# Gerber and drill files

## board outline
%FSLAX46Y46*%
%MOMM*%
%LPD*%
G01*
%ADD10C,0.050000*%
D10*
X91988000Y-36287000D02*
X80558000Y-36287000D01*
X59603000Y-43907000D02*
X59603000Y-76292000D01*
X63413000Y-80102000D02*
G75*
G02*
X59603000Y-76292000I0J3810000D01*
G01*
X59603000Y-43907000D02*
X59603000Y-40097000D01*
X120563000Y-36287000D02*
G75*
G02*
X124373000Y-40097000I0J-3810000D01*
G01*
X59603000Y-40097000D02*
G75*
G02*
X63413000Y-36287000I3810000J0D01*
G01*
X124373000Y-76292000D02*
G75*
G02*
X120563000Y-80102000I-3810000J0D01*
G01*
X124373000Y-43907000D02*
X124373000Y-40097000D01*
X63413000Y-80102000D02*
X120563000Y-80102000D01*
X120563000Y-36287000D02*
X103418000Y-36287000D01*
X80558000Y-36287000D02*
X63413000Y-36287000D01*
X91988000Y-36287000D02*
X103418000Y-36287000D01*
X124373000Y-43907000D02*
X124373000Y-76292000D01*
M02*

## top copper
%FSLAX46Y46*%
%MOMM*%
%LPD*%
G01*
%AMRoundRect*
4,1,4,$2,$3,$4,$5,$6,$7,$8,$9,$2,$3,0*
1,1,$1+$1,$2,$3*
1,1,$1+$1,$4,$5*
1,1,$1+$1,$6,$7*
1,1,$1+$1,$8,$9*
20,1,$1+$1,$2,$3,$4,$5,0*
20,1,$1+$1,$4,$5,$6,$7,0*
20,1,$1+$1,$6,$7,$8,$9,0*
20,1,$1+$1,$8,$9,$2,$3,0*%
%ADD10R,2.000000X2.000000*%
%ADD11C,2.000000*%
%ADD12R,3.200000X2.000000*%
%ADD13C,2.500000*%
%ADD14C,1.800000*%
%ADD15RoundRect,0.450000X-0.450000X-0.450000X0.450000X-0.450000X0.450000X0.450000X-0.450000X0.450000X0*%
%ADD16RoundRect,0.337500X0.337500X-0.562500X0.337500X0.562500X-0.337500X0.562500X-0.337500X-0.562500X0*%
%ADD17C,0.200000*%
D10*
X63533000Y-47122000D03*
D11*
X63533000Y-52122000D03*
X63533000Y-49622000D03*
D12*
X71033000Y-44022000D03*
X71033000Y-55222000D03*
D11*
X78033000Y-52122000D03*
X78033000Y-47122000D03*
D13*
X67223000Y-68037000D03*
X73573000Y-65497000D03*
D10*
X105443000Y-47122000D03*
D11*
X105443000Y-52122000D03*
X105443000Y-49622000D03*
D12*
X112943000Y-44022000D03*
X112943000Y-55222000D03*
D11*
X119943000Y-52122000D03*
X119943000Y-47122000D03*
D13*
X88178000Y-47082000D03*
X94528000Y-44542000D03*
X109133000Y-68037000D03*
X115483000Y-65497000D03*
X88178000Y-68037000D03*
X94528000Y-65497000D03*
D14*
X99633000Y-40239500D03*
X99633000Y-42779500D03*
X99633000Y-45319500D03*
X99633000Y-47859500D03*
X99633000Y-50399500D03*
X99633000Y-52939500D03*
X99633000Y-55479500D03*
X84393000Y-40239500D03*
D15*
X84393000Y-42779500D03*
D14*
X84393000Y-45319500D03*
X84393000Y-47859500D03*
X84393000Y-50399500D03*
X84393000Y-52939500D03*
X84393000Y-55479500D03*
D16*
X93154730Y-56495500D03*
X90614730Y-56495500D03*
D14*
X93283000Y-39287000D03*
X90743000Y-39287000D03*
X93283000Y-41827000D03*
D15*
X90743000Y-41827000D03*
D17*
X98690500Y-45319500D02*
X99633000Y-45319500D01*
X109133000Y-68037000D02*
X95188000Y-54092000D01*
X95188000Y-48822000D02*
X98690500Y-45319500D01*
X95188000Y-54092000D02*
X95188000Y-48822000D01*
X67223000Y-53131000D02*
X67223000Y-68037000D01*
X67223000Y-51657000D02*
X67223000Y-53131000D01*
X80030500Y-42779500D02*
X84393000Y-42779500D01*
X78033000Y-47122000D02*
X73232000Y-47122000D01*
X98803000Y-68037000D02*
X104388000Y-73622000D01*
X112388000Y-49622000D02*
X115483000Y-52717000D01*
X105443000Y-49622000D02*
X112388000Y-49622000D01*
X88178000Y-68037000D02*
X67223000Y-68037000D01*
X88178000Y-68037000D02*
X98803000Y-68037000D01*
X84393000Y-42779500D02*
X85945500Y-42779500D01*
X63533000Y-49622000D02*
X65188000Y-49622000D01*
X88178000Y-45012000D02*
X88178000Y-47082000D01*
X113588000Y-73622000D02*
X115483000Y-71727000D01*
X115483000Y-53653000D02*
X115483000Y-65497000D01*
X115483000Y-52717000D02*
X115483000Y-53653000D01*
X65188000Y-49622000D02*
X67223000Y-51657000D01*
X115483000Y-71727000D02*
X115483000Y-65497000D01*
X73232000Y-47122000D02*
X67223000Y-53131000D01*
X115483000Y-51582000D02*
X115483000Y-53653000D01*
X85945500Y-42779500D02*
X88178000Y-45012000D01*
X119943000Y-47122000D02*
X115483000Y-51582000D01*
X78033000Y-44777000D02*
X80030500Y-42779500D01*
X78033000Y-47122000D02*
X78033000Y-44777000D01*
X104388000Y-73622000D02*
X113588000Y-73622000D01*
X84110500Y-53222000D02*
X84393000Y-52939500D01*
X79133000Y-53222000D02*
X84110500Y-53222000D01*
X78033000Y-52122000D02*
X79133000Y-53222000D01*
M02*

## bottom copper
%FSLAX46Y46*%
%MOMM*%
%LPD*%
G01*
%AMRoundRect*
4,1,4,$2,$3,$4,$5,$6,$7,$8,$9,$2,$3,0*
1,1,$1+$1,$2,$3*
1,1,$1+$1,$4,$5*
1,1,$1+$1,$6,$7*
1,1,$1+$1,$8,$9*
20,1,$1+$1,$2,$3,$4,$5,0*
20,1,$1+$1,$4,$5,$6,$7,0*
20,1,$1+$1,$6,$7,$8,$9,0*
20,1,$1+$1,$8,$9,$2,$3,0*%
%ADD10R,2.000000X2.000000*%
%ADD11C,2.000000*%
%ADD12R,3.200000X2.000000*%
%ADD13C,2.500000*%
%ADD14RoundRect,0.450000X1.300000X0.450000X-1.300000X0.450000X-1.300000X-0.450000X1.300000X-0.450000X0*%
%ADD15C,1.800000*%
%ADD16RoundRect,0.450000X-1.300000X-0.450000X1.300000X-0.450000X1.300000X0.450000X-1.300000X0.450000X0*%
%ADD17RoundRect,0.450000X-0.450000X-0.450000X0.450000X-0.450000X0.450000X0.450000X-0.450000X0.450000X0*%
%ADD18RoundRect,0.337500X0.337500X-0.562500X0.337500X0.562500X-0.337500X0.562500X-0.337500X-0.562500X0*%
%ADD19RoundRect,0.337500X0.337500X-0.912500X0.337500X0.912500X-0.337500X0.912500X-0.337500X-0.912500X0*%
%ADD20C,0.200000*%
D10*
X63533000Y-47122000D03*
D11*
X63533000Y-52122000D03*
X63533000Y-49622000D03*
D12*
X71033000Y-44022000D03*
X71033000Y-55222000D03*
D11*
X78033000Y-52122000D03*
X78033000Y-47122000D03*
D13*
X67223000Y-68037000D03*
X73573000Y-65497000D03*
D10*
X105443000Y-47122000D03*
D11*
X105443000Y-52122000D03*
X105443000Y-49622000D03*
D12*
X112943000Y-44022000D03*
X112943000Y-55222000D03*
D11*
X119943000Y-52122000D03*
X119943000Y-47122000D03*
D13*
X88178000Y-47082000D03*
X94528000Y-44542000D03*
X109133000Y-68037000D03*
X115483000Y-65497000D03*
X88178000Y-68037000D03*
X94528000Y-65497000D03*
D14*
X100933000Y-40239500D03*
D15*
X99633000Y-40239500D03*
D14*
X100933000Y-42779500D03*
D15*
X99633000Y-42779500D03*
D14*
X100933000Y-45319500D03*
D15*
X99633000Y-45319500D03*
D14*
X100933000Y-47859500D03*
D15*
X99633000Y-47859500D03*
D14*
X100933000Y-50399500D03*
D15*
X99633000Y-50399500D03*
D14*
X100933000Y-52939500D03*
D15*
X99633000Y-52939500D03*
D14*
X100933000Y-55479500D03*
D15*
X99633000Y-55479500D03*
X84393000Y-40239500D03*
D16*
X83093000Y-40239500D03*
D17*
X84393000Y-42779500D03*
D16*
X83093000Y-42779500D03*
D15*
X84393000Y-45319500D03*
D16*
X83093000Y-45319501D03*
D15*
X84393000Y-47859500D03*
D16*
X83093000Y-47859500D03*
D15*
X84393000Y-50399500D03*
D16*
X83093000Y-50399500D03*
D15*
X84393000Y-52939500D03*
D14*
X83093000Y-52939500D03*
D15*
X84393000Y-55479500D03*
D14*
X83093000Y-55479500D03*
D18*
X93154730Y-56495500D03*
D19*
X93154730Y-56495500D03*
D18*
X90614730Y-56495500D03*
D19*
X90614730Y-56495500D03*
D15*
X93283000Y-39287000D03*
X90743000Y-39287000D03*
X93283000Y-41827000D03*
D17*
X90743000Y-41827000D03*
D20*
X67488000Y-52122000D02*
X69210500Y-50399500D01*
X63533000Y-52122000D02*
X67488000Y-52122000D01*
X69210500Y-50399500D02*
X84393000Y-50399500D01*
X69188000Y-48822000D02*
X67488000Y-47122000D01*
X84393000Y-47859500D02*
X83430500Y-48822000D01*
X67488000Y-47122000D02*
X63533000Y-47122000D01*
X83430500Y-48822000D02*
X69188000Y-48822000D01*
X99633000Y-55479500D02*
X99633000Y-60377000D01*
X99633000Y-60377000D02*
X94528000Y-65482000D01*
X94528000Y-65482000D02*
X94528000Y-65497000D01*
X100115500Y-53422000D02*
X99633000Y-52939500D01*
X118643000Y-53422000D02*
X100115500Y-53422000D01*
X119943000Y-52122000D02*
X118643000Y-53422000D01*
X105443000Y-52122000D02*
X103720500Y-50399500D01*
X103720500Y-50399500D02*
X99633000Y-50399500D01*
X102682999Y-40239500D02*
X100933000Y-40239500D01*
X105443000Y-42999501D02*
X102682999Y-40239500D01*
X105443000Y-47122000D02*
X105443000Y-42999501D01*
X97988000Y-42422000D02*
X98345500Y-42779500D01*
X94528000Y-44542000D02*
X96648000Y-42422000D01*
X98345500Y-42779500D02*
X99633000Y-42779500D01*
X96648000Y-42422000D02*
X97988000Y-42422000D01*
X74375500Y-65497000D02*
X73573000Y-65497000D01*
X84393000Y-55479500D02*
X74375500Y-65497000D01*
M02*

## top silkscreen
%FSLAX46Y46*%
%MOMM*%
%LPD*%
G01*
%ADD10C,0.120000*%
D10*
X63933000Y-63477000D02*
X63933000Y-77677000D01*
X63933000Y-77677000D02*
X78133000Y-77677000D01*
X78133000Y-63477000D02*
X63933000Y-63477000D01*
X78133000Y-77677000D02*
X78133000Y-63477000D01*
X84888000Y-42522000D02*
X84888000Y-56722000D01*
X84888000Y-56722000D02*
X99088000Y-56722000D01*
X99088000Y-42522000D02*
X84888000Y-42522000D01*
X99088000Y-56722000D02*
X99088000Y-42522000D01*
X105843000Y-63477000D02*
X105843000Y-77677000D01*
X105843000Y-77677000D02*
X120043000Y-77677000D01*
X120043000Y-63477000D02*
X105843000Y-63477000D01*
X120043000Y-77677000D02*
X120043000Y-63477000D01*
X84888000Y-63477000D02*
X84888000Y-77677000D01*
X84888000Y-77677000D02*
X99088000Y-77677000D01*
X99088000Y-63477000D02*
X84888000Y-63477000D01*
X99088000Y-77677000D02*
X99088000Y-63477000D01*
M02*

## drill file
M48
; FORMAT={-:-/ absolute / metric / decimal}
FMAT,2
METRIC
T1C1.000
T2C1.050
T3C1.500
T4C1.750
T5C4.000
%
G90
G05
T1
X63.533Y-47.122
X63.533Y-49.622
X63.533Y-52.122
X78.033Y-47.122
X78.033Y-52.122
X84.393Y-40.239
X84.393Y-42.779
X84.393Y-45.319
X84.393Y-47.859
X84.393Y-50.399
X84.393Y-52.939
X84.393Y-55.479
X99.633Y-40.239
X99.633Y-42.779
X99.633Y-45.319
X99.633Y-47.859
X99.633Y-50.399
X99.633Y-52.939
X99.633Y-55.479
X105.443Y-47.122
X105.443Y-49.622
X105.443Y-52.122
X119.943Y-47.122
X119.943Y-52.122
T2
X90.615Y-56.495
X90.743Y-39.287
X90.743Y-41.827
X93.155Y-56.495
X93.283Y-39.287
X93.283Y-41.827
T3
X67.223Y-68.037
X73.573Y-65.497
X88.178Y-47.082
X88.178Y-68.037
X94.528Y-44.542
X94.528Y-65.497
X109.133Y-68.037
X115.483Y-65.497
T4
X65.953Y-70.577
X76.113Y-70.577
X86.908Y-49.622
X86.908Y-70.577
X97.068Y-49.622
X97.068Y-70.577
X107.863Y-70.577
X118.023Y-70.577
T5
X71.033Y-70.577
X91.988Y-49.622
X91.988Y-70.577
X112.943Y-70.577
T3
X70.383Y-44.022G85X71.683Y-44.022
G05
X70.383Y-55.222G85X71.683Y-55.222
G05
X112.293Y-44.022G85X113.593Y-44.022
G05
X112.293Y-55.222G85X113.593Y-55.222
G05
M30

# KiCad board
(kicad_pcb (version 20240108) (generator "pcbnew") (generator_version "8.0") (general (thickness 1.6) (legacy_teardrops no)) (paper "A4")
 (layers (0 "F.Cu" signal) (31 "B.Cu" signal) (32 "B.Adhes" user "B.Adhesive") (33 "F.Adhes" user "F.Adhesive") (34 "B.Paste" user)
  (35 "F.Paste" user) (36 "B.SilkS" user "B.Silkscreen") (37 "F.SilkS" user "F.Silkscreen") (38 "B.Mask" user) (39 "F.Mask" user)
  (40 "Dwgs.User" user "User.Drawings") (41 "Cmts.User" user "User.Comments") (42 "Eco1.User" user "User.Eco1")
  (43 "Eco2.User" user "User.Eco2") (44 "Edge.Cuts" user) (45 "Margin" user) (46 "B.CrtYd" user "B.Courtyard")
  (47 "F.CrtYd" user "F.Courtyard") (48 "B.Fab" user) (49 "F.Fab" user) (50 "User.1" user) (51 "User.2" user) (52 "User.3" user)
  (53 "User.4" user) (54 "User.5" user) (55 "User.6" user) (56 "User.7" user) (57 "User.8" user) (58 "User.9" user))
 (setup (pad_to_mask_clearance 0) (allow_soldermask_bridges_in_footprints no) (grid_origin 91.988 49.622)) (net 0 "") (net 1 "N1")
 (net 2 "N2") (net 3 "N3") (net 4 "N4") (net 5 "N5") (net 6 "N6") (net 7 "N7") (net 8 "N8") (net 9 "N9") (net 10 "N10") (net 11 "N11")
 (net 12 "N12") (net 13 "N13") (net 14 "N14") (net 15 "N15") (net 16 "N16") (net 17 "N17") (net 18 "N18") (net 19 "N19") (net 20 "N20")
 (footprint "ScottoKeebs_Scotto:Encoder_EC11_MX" (layer "F.Cu") (at 71.033 49.622)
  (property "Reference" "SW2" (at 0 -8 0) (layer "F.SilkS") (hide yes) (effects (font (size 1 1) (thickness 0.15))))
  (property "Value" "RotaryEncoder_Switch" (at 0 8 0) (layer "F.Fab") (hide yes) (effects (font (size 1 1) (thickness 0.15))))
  (pad "A" thru_hole rect (at -7.5 -2.5) (size 2 2) (drill 1) (layers "*.Cu" "*.Mask") (remove_unused_layers no) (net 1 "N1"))
  (pad "B" thru_hole circle (at -7.5 2.5) (size 2 2) (drill 1) (layers "*.Cu" "*.Mask") (remove_unused_layers no) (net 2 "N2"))
  (pad "C" thru_hole circle (at -7.5 0) (size 2 2) (drill 1) (layers "*.Cu" "*.Mask") (remove_unused_layers no) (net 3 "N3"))
  (pad "MP" thru_hole rect (at 0 -5.6) (size 3.2 2) (drill oval 2.8 1.5) (layers "*.Cu" "*.Mask") (remove_unused_layers no))
  (pad "MP" thru_hole rect (at 0 5.6) (size 3.2 2) (drill oval 2.8 1.5) (layers "*.Cu" "*.Mask") (remove_unused_layers no))
  (pad "S1" thru_hole circle (at 7 2.5) (size 2 2) (drill 1) (layers "*.Cu" "*.Mask") (remove_unused_layers no) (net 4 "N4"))
  (pad "S2" thru_hole circle (at 7 -2.5) (size 2 2) (drill 1) (layers "*.Cu" "*.Mask") (remove_unused_layers no) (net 3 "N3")))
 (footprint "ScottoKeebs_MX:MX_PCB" (layer "F.Cu") (at 71.033 70.577)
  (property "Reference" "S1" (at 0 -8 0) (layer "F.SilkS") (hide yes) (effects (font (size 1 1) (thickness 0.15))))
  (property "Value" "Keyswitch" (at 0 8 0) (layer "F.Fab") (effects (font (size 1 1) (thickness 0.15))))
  (fp_line (start -7.1 -7.1) (end -7.1 7.1) (stroke (width 0.12) (type solid)) (layer "F.SilkS"))
  (fp_line (start -7.1 7.1) (end 7.1 7.1) (stroke (width 0.12) (type solid)) (layer "F.SilkS"))
  (fp_line (start 7.1 -7.1) (end -7.1 -7.1) (stroke (width 0.12) (type solid)) (layer "F.SilkS"))
  (fp_line (start 7.1 7.1) (end 7.1 -7.1) (stroke (width 0.12) (type solid)) (layer "F.SilkS"))
  (pad "" np_thru_hole circle (at -5.08 0) (size 1.75 1.75) (drill 1.75) (layers "*.Cu" "*.Mask"))
  (pad "" np_thru_hole circle (at 0 0) (size 4 4) (drill 4) (layers "*.Cu" "*.Mask"))
  (pad "" np_thru_hole circle (at 5.08 0) (size 1.75 1.75) (drill 1.75) (layers "*.Cu" "*.Mask"))
  (pad "1" thru_hole circle (at -3.81 -2.54) (size 2.5 2.5) (drill 1.5) (layers "*.Cu" "*.Mask") (remove_unused_layers no) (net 3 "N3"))
  (pad "2" thru_hole circle (at 2.54 -5.08) (size 2.5 2.5) (drill 1.5) (layers "*.Cu" "*.Mask") (remove_unused_layers no) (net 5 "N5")))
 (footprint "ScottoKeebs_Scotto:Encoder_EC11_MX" (layer "F.Cu") (at 112.943 49.622)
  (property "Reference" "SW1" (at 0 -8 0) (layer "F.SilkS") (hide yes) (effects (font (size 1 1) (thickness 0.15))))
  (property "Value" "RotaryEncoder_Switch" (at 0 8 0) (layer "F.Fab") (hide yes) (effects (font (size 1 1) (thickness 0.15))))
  (pad "A" thru_hole rect (at -7.5 -2.5) (size 2 2) (drill 1) (layers "*.Cu" "*.Mask") (remove_unused_layers no) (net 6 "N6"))
  (pad "B" thru_hole circle (at -7.5 2.5) (size 2 2) (drill 1) (layers "*.Cu" "*.Mask") (remove_unused_layers no) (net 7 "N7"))
  (pad "C" thru_hole circle (at -7.5 0) (size 2 2) (drill 1) (layers "*.Cu" "*.Mask") (remove_unused_layers no) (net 3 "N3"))
  (pad "MP" thru_hole rect (at 0 -5.6) (size 3.2 2) (drill oval 2.8 1.5) (layers "*.Cu" "*.Mask") (remove_unused_layers no))
  (pad "MP" thru_hole rect (at 0 5.6) (size 3.2 2) (drill oval 2.8 1.5) (layers "*.Cu" "*.Mask") (remove_unused_layers no))
  (pad "S1" thru_hole circle (at 7 2.5) (size 2 2) (drill 1) (layers "*.Cu" "*.Mask") (remove_unused_layers no) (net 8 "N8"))
  (pad "S2" thru_hole circle (at 7 -2.5) (size 2 2) (drill 1) (layers "*.Cu" "*.Mask") (remove_unused_layers no) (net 3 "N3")))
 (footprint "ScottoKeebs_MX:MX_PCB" (layer "F.Cu") (at 91.988 49.622)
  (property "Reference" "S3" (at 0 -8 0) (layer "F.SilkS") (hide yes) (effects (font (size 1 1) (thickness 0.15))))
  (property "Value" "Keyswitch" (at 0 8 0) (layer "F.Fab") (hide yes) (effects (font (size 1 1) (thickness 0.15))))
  (fp_line (start -7.1 -7.1) (end -7.1 7.1) (stroke (width 0.12) (type solid)) (layer "F.SilkS"))
  (fp_line (start -7.1 7.1) (end 7.1 7.1) (stroke (width 0.12) (type solid)) (layer "F.SilkS"))
  (fp_line (start 7.1 -7.1) (end -7.1 -7.1) (stroke (width 0.12) (type solid)) (layer "F.SilkS"))
  (fp_line (start 7.1 7.1) (end 7.1 -7.1) (stroke (width 0.12) (type solid)) (layer "F.SilkS"))
  (pad "" np_thru_hole circle (at -5.08 0) (size 1.75 1.75) (drill 1.75) (layers "*.Cu" "*.Mask"))
  (pad "" np_thru_hole circle (at 0 0) (size 4 4) (drill 4) (layers "*.Cu" "*.Mask"))
  (pad "" np_thru_hole circle (at 5.08 0) (size 1.75 1.75) (drill 1.75) (layers "*.Cu" "*.Mask"))
  (pad "1" thru_hole circle (at -3.81 -2.54) (size 2.5 2.5) (drill 1.5) (layers "*.Cu" "*.Mask") (remove_unused_layers no) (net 3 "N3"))
  (pad "2" thru_hole circle (at 2.54 -5.08) (size 2.5 2.5) (drill 1.5) (layers "*.Cu" "*.Mask") (remove_unused_layers no) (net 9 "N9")))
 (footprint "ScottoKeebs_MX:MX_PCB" (layer "F.Cu") (at 112.943 70.577)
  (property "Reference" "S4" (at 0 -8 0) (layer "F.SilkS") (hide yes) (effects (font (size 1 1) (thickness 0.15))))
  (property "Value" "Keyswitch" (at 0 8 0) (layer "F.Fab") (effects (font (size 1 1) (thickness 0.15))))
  (fp_line (start -7.1 -7.1) (end -7.1 7.1) (stroke (width 0.12) (type solid)) (layer "F.SilkS"))
  (fp_line (start -7.1 7.1) (end 7.1 7.1) (stroke (width 0.12) (type solid)) (layer "F.SilkS"))
  (fp_line (start 7.1 -7.1) (end -7.1 -7.1) (stroke (width 0.12) (type solid)) (layer "F.SilkS"))
  (fp_line (start 7.1 7.1) (end 7.1 -7.1) (stroke (width 0.12) (type solid)) (layer "F.SilkS"))
  (pad "" np_thru_hole circle (at -5.08 0) (size 1.75 1.75) (drill 1.75) (layers "*.Cu" "*.Mask"))
  (pad "" np_thru_hole circle (at 0 0) (size 4 4) (drill 4) (layers "*.Cu" "*.Mask"))
  (pad "" np_thru_hole circle (at 5.08 0) (size 1.75 1.75) (drill 1.75) (layers "*.Cu" "*.Mask"))
  (pad "1" thru_hole circle (at -3.81 -2.54) (size 2.5 2.5) (drill 1.5) (layers "*.Cu" "*.Mask") (remove_unused_layers no) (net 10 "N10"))
  (pad "2" thru_hole circle (at 2.54 -5.08) (size 2.5 2.5) (drill 1.5) (layers "*.Cu" "*.Mask") (remove_unused_layers no) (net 3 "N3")))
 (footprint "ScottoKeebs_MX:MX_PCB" (layer "F.Cu") (at 91.988 70.577)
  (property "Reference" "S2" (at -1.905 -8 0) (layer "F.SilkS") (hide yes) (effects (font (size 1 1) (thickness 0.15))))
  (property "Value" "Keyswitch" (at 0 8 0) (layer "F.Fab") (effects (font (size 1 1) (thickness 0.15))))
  (fp_line (start -7.1 -7.1) (end -7.1 7.1) (stroke (width 0.12) (type solid)) (layer "F.SilkS"))
  (fp_line (start -7.1 7.1) (end 7.1 7.1) (stroke (width 0.12) (type solid)) (layer "F.SilkS"))
  (fp_line (start 7.1 -7.1) (end -7.1 -7.1) (stroke (width 0.12) (type solid)) (layer "F.SilkS"))
  (fp_line (start 7.1 7.1) (end 7.1 -7.1) (stroke (width 0.12) (type solid)) (layer "F.SilkS"))
  (pad "" np_thru_hole circle (at -5.08 0) (size 1.75 1.75) (drill 1.75) (layers "*.Cu" "*.Mask"))
  (pad "" np_thru_hole circle (at 0 0) (size 4 4) (drill 4) (layers "*.Cu" "*.Mask"))
  (pad "" np_thru_hole circle (at 5.08 0) (size 1.75 1.75) (drill 1.75) (layers "*.Cu" "*.Mask"))
  (pad "1" thru_hole circle (at -3.81 -2.54) (size 2.5 2.5) (drill 1.5) (layers "*.Cu" "*.Mask") (remove_unused_layers no) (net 3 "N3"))
  (pad "2" thru_hole circle (at 2.54 -5.08) (size 2.5 2.5) (drill 1.5) (layers "*.Cu" "*.Mask") (remove_unused_layers no) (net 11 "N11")))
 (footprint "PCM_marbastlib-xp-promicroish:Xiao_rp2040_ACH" (layer "B.Cu") (at 92.013 47.8595 180)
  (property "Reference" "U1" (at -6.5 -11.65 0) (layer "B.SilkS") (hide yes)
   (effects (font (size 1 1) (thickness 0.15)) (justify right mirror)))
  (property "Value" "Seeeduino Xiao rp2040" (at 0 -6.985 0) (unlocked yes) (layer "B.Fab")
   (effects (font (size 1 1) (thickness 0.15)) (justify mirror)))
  (pad "1" smd roundrect (at -8.92 7.62 180) (size 3.5 1.8) (layers "B.Cu" "B.Mask") (roundrect_rratio 0.25) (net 6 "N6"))
  (pad "1" thru_hole circle (at -7.62 7.62 180) (size 1.8 1.8) (drill 1) (layers "*.Cu" "*.Mask") (remove_unused_layers no) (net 6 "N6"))
  (pad "2" smd roundrect (at -8.92 5.08 180) (size 3.5 1.8) (layers "B.Cu" "B.Mask") (roundrect_rratio 0.25) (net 9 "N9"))
  (pad "2" thru_hole circle (at -7.62 5.08 180) (size 1.8 1.8) (drill 1) (layers "*.Cu" "*.Mask") (remove_unused_layers no) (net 9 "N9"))
  (pad "3" smd roundrect (at -8.92 2.54 180) (size 3.5 1.8) (layers "B.Cu" "B.Mask") (roundrect_rratio 0.25) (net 10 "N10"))
  (pad "3" thru_hole circle (at -7.62 2.54 180) (size 1.8 1.8) (drill 1) (layers "*.Cu" "*.Mask") (remove_unused_layers no) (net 10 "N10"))
  (pad "4" smd roundrect (at -8.92 0 180) (size 3.5 1.8) (layers "B.Cu" "B.Mask") (roundrect_rratio 0.25) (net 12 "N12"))
  (pad "4" thru_hole circle (at -7.62 0 180) (size 1.8 1.8) (drill 1) (layers "*.Cu" "*.Mask") (remove_unused_layers no) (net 12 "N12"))
  (pad "5" smd roundrect (at -8.92 -2.54 180) (size 3.5 1.8) (layers "B.Cu" "B.Mask") (roundrect_rratio 0.25) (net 7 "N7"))
  (pad "5" thru_hole circle (at -7.62 -2.54 180) (size 1.8 1.8) (drill 1) (layers "*.Cu" "*.Mask") (remove_unused_layers no) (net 7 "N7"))
  (pad "6" smd roundrect (at -8.92 -5.08 180) (size 3.5 1.8) (layers "B.Cu" "B.Mask") (roundrect_rratio 0.25) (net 8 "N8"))
  (pad "6" thru_hole circle (at -7.62 -5.08 180) (size 1.8 1.8) (drill 1) (layers "*.Cu" "*.Mask") (remove_unused_layers no) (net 8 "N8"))
  (pad "7" smd roundrect (at -8.92 -7.62 180) (size 3.5 1.8) (layers "B.Cu" "B.Mask") (roundrect_rratio 0.25) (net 11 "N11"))
  (pad "7" thru_hole circle (at -7.62 -7.62 180) (size 1.8 1.8) (drill 1) (layers "*.Cu" "*.Mask") (remove_unused_layers no) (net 11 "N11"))
  (pad "8" thru_hole circle (at 7.62 7.62) (size 1.8 1.8) (drill 1) (layers "*.Cu" "*.Mask") (remove_unused_layers no) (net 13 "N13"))
  (pad "8" smd roundrect (at 8.92 7.62) (size 3.5 1.8) (layers "B.Cu" "B.Mask") (roundrect_rratio 0.25) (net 13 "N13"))
  (pad "9" thru_hole roundrect (at 7.62 5.08) (size 1.8 1.8) (drill 1) (layers "*.Cu" "*.Mask") (remove_unused_layers no)
   (roundrect_rratio 0.25) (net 3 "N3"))
  (pad "9" smd roundrect (at 8.92 5.08) (size 3.5 1.8) (layers "B.Cu" "B.Mask") (roundrect_rratio 0.25) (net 3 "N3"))
  (pad "10" thru_hole circle (at 7.62 2.54) (size 1.8 1.8) (drill 1) (layers "*.Cu" "*.Mask") (remove_unused_layers no) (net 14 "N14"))
  (pad "10" smd roundrect (at 8.92 2.539999) (size 3.5 1.8) (layers "B.Cu" "B.Mask") (roundrect_rratio 0.25) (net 14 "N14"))
  (pad "11" thru_hole circle (at 7.62 0) (size 1.8 1.8) (drill 1) (layers "*.Cu" "*.Mask") (remove_unused_layers no) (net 1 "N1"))
  (pad "11" smd roundrect (at 8.92 0) (size 3.5 1.8) (layers "B.Cu" "B.Mask") (roundrect_rratio 0.25) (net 1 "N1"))
  (pad "12" thru_hole circle (at 7.62 -2.54) (size 1.8 1.8) (drill 1) (layers "*.Cu" "*.Mask") (remove_unused_layers no) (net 2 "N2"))
  (pad "12" smd roundrect (at 8.92 -2.54) (size 3.5 1.8) (layers "B.Cu" "B.Mask") (roundrect_rratio 0.25) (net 2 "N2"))
  (pad "13" thru_hole circle (at 7.62 -5.08 180) (size 1.8 1.8) (drill 1) (layers "*.Cu" "*.Mask") (remove_unused_layers no) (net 4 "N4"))
  (pad "13" smd roundrect (at 8.92 -5.08 180) (size 3.5 1.8) (layers "B.Cu" "B.Mask") (roundrect_rratio 0.25) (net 4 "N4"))
  (pad "14" thru_hole circle (at 7.62 -7.62 180) (size 1.8 1.8) (drill 1) (layers "*.Cu" "*.Mask") (remove_unused_layers no) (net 5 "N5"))
  (pad "14" smd roundrect (at 8.92 -7.62 180) (size 3.5 1.8) (layers "B.Cu" "B.Mask") (roundrect_rratio 0.25) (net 5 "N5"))
  (pad "17" thru_hole roundrect (at -1.14173 -8.636 90) (size 1.8 1.35) (drill 1.05) (layers "*.Cu" "*.Mask") (remove_unused_layers no)
   (roundrect_rratio 0.25) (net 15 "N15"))
  (pad "17" smd roundrect (at -1.14173 -8.636 90) (size 2.5 1.35) (layers "B.Cu" "B.Mask") (roundrect_rratio 0.25) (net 15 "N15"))
  (pad "18" thru_hole roundrect (at 1.39827 -8.636 90) (size 1.8 1.35) (drill 1.05) (layers "*.Cu" "*.Mask") (remove_unused_layers no)
   (roundrect_rratio 0.25) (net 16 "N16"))
  (pad "18" smd roundrect (at 1.39827 -8.636 90) (size 2.5 1.35) (layers "B.Cu" "B.Mask") (roundrect_rratio 0.25) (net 16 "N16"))
  (pad "19" thru_hole circle (at -1.27 8.5725) (size 1.8 1.8) (drill 1.05) (layers "*.Cu" "*.Mask") (remove_unused_layers no) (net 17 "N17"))
  (pad "20" thru_hole circle (at 1.27 8.5725) (size 1.8 1.8) (drill 1.05) (layers "*.Cu" "*.Mask") (remove_unused_layers no) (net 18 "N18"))
  (pad "21" thru_hole circle (at -1.27 6.0325) (size 1.8 1.8) (drill 1.05) (layers "*.Cu" "*.Mask") (remove_unused_layers no) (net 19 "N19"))
  (pad "22" thru_hole roundrect (at 1.27 6.0325) (size 1.8 1.8) (drill 1.05) (layers "*.Cu" "*.Mask") (remove_unused_layers no)
   (roundrect_rratio 0.25) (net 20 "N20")))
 (gr_line (start 91.988 36.287) (end 80.558 36.287) (stroke (width 0.05) (type default)) (layer "Edge.Cuts"))
 (gr_line (start 59.603 43.907) (end 59.603 76.292) (stroke (width 0.05) (type default)) (layer "Edge.Cuts"))
 (gr_arc (start 63.413 80.102) (mid 60.718923 78.986077) (end 59.603 76.292) (stroke (width 0.05) (type default)) (layer "Edge.Cuts"))
 (gr_line (start 59.603 43.907) (end 59.603 40.097) (stroke (width 0.05) (type default)) (layer "Edge.Cuts"))
 (gr_arc (start 120.563 36.287) (mid 123.257077 37.402923) (end 124.373 40.097) (stroke (width 0.05) (type default)) (layer "Edge.Cuts"))
 (gr_arc (start 59.603 40.097) (mid 60.718923 37.402923) (end 63.413 36.287) (stroke (width 0.05) (type default)) (layer "Edge.Cuts"))
 (gr_arc (start 124.373 76.292) (mid 123.257077 78.986077) (end 120.563 80.102) (stroke (width 0.05) (type default)) (layer "Edge.Cuts"))
 (gr_line (start 124.373 43.907) (end 124.373 40.097) (stroke (width 0.05) (type default)) (layer "Edge.Cuts"))
 (gr_line (start 63.413 80.102) (end 120.563 80.102) (stroke (width 0.05) (type default)) (layer "Edge.Cuts"))
 (gr_line (start 120.563 36.287) (end 103.418 36.287) (stroke (width 0.05) (type default)) (layer "Edge.Cuts"))
 (gr_line (start 80.558 36.287) (end 63.413 36.287) (stroke (width 0.05) (type default)) (layer "Edge.Cuts"))
 (gr_line (start 91.988 36.287) (end 103.418 36.287) (stroke (width 0.05) (type default)) (layer "Edge.Cuts"))
 (gr_line (start 124.373 43.907) (end 124.373 76.292) (stroke (width 0.05) (type default)) (layer "Edge.Cuts"))
 (segment (start 67.488 52.122) (end 69.2105 50.3995) (width 0.2) (layer "B.Cu") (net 2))
 (segment (start 63.533 52.122) (end 67.488 52.122) (width 0.2) (layer "B.Cu") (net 2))
 (segment (start 69.2105 50.3995) (end 84.393 50.3995) (width 0.2) (layer "B.Cu") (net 2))
 (segment (start 69.188 48.822) (end 67.488 47.122) (width 0.2) (layer "B.Cu") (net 1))
 (segment (start 84.393 47.8595) (end 83.4305 48.822) (width 0.2) (layer "B.Cu") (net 1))
 (segment (start 67.488 47.122) (end 63.533 47.122) (width 0.2) (layer "B.Cu") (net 1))
 (segment (start 83.4305 48.822) (end 69.188 48.822) (width 0.2) (layer "B.Cu") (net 1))
 (segment (start 99.633 55.4795) (end 99.633 60.377) (width 0.2) (layer "B.Cu") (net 11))
 (segment (start 99.633 60.377) (end 94.528 65.482) (width 0.2) (layer "B.Cu") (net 11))
 (segment (start 94.528 65.482) (end 94.528 65.497) (width 0.2) (layer "B.Cu") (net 11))
 (segment (start 98.6905 45.3195) (end 99.633 45.3195) (width 0.2) (layer "F.Cu") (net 10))
 (segment (start 109.133 68.037) (end 95.188 54.092) (width 0.2) (layer "F.Cu") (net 10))
 (segment (start 95.188 48.822) (end 98.6905 45.3195) (width 0.2) (layer "F.Cu") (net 10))
 (segment (start 95.188 54.092) (end 95.188 48.822) (width 0.2) (layer "F.Cu") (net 10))
 (segment (start 100.1155 53.422) (end 99.633 52.9395) (width 0.2) (layer "B.Cu") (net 8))
 (segment (start 118.643 53.422) (end 100.1155 53.422) (width 0.2) (layer "B.Cu") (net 8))
 (segment (start 119.943 52.122) (end 118.643 53.422) (width 0.2) (layer "B.Cu") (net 8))
 (segment (start 105.443 52.122) (end 103.7205 50.3995) (width 0.2) (layer "B.Cu") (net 7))
 (segment (start 103.7205 50.3995) (end 99.633 50.3995) (width 0.2) (layer "B.Cu") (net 7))
 (segment (start 67.223 53.131) (end 67.223 68.037) (width 0.2) (layer "F.Cu") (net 3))
 (segment (start 67.223 51.657) (end 67.223 53.131) (width 0.2) (layer "F.Cu") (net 3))
 (segment (start 80.0305 42.7795) (end 84.393 42.7795) (width 0.2) (layer "F.Cu") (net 3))
 (segment (start 78.033 47.122) (end 73.232 47.122) (width 0.2) (layer "F.Cu") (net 3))
 (segment (start 98.803 68.037) (end 104.388 73.622) (width 0.2) (layer "F.Cu") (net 3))
 (segment (start 112.388 49.622) (end 115.483 52.717) (width 0.2) (layer "F.Cu") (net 3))
 (segment (start 105.443 49.622) (end 112.388 49.622) (width 0.2) (layer "F.Cu") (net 3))
 (segment (start 88.178 68.037) (end 67.223 68.037) (width 0.2) (layer "F.Cu") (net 3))
 (segment (start 88.178 68.037) (end 98.803 68.037) (width 0.2) (layer "F.Cu") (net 3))
 (segment (start 84.393 42.7795) (end 85.9455 42.7795) (width 0.2) (layer "F.Cu") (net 3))
 (segment (start 63.533 49.622) (end 65.188 49.622) (width 0.2) (layer "F.Cu") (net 3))
 (segment (start 88.178 45.012) (end 88.178 47.082) (width 0.2) (layer "F.Cu") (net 3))
 (segment (start 113.588 73.622) (end 115.483 71.727) (width 0.2) (layer "F.Cu") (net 3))
 (segment (start 115.483 53.653) (end 115.483 65.497) (width 0.2) (layer "F.Cu") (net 3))
 (segment (start 115.483 52.717) (end 115.483 53.653) (width 0.2) (layer "F.Cu") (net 3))
 (segment (start 65.188 49.622) (end 67.223 51.657) (width 0.2) (layer "F.Cu") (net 3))
 (segment (start 115.483 71.727) (end 115.483 65.497) (width 0.2) (layer "F.Cu") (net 3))
 (segment (start 73.232 47.122) (end 67.223 53.131) (width 0.2) (layer "F.Cu") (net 3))
 (segment (start 115.483 51.582) (end 115.483 53.653) (width 0.2) (layer "F.Cu") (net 3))
 (segment (start 85.9455 42.7795) (end 88.178 45.012) (width 0.2) (layer "F.Cu") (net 3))
 (segment (start 119.943 47.122) (end 115.483 51.582) (width 0.2) (layer "F.Cu") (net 3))
 (segment (start 78.033 44.777) (end 80.0305 42.7795) (width 0.2) (layer "F.Cu") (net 3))
 (segment (start 78.033 47.122) (end 78.033 44.777) (width 0.2) (layer "F.Cu") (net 3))
 (segment (start 104.388 73.622) (end 113.588 73.622) (width 0.2) (layer "F.Cu") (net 3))
 (segment (start 102.682999 40.2395) (end 100.933 40.2395) (width 0.2) (layer "B.Cu") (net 6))
 (segment (start 105.443 42.999501) (end 102.682999 40.2395) (width 0.2) (layer "B.Cu") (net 6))
 (segment (start 105.443 47.122) (end 105.443 42.999501) (width 0.2) (layer "B.Cu") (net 6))
 (segment (start 97.988 42.422) (end 98.3455 42.7795) (width 0.2) (layer "B.Cu") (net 9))
 (segment (start 94.528 44.542) (end 96.648 42.422) (width 0.2) (layer "B.Cu") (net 9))
 (segment (start 98.3455 42.7795) (end 99.633 42.7795) (width 0.2) (layer "B.Cu") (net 9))
 (segment (start 96.648 42.422) (end 97.988 42.422) (width 0.2) (layer "B.Cu") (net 9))
 (segment (start 84.1105 53.222) (end 84.393 52.9395) (width 0.2) (layer "F.Cu") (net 4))
 (segment (start 79.133 53.222) (end 84.1105 53.222) (width 0.2) (layer "F.Cu") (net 4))
 (segment (start 78.033 52.122) (end 79.133 53.222) (width 0.2) (layer "F.Cu") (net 4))
 (segment (start 74.3755 65.497) (end 73.573 65.497) (width 0.2) (layer "B.Cu") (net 5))
 (segment (start 84.393 55.4795) (end 74.3755 65.497) (width 0.2) (layer "B.Cu") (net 5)))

